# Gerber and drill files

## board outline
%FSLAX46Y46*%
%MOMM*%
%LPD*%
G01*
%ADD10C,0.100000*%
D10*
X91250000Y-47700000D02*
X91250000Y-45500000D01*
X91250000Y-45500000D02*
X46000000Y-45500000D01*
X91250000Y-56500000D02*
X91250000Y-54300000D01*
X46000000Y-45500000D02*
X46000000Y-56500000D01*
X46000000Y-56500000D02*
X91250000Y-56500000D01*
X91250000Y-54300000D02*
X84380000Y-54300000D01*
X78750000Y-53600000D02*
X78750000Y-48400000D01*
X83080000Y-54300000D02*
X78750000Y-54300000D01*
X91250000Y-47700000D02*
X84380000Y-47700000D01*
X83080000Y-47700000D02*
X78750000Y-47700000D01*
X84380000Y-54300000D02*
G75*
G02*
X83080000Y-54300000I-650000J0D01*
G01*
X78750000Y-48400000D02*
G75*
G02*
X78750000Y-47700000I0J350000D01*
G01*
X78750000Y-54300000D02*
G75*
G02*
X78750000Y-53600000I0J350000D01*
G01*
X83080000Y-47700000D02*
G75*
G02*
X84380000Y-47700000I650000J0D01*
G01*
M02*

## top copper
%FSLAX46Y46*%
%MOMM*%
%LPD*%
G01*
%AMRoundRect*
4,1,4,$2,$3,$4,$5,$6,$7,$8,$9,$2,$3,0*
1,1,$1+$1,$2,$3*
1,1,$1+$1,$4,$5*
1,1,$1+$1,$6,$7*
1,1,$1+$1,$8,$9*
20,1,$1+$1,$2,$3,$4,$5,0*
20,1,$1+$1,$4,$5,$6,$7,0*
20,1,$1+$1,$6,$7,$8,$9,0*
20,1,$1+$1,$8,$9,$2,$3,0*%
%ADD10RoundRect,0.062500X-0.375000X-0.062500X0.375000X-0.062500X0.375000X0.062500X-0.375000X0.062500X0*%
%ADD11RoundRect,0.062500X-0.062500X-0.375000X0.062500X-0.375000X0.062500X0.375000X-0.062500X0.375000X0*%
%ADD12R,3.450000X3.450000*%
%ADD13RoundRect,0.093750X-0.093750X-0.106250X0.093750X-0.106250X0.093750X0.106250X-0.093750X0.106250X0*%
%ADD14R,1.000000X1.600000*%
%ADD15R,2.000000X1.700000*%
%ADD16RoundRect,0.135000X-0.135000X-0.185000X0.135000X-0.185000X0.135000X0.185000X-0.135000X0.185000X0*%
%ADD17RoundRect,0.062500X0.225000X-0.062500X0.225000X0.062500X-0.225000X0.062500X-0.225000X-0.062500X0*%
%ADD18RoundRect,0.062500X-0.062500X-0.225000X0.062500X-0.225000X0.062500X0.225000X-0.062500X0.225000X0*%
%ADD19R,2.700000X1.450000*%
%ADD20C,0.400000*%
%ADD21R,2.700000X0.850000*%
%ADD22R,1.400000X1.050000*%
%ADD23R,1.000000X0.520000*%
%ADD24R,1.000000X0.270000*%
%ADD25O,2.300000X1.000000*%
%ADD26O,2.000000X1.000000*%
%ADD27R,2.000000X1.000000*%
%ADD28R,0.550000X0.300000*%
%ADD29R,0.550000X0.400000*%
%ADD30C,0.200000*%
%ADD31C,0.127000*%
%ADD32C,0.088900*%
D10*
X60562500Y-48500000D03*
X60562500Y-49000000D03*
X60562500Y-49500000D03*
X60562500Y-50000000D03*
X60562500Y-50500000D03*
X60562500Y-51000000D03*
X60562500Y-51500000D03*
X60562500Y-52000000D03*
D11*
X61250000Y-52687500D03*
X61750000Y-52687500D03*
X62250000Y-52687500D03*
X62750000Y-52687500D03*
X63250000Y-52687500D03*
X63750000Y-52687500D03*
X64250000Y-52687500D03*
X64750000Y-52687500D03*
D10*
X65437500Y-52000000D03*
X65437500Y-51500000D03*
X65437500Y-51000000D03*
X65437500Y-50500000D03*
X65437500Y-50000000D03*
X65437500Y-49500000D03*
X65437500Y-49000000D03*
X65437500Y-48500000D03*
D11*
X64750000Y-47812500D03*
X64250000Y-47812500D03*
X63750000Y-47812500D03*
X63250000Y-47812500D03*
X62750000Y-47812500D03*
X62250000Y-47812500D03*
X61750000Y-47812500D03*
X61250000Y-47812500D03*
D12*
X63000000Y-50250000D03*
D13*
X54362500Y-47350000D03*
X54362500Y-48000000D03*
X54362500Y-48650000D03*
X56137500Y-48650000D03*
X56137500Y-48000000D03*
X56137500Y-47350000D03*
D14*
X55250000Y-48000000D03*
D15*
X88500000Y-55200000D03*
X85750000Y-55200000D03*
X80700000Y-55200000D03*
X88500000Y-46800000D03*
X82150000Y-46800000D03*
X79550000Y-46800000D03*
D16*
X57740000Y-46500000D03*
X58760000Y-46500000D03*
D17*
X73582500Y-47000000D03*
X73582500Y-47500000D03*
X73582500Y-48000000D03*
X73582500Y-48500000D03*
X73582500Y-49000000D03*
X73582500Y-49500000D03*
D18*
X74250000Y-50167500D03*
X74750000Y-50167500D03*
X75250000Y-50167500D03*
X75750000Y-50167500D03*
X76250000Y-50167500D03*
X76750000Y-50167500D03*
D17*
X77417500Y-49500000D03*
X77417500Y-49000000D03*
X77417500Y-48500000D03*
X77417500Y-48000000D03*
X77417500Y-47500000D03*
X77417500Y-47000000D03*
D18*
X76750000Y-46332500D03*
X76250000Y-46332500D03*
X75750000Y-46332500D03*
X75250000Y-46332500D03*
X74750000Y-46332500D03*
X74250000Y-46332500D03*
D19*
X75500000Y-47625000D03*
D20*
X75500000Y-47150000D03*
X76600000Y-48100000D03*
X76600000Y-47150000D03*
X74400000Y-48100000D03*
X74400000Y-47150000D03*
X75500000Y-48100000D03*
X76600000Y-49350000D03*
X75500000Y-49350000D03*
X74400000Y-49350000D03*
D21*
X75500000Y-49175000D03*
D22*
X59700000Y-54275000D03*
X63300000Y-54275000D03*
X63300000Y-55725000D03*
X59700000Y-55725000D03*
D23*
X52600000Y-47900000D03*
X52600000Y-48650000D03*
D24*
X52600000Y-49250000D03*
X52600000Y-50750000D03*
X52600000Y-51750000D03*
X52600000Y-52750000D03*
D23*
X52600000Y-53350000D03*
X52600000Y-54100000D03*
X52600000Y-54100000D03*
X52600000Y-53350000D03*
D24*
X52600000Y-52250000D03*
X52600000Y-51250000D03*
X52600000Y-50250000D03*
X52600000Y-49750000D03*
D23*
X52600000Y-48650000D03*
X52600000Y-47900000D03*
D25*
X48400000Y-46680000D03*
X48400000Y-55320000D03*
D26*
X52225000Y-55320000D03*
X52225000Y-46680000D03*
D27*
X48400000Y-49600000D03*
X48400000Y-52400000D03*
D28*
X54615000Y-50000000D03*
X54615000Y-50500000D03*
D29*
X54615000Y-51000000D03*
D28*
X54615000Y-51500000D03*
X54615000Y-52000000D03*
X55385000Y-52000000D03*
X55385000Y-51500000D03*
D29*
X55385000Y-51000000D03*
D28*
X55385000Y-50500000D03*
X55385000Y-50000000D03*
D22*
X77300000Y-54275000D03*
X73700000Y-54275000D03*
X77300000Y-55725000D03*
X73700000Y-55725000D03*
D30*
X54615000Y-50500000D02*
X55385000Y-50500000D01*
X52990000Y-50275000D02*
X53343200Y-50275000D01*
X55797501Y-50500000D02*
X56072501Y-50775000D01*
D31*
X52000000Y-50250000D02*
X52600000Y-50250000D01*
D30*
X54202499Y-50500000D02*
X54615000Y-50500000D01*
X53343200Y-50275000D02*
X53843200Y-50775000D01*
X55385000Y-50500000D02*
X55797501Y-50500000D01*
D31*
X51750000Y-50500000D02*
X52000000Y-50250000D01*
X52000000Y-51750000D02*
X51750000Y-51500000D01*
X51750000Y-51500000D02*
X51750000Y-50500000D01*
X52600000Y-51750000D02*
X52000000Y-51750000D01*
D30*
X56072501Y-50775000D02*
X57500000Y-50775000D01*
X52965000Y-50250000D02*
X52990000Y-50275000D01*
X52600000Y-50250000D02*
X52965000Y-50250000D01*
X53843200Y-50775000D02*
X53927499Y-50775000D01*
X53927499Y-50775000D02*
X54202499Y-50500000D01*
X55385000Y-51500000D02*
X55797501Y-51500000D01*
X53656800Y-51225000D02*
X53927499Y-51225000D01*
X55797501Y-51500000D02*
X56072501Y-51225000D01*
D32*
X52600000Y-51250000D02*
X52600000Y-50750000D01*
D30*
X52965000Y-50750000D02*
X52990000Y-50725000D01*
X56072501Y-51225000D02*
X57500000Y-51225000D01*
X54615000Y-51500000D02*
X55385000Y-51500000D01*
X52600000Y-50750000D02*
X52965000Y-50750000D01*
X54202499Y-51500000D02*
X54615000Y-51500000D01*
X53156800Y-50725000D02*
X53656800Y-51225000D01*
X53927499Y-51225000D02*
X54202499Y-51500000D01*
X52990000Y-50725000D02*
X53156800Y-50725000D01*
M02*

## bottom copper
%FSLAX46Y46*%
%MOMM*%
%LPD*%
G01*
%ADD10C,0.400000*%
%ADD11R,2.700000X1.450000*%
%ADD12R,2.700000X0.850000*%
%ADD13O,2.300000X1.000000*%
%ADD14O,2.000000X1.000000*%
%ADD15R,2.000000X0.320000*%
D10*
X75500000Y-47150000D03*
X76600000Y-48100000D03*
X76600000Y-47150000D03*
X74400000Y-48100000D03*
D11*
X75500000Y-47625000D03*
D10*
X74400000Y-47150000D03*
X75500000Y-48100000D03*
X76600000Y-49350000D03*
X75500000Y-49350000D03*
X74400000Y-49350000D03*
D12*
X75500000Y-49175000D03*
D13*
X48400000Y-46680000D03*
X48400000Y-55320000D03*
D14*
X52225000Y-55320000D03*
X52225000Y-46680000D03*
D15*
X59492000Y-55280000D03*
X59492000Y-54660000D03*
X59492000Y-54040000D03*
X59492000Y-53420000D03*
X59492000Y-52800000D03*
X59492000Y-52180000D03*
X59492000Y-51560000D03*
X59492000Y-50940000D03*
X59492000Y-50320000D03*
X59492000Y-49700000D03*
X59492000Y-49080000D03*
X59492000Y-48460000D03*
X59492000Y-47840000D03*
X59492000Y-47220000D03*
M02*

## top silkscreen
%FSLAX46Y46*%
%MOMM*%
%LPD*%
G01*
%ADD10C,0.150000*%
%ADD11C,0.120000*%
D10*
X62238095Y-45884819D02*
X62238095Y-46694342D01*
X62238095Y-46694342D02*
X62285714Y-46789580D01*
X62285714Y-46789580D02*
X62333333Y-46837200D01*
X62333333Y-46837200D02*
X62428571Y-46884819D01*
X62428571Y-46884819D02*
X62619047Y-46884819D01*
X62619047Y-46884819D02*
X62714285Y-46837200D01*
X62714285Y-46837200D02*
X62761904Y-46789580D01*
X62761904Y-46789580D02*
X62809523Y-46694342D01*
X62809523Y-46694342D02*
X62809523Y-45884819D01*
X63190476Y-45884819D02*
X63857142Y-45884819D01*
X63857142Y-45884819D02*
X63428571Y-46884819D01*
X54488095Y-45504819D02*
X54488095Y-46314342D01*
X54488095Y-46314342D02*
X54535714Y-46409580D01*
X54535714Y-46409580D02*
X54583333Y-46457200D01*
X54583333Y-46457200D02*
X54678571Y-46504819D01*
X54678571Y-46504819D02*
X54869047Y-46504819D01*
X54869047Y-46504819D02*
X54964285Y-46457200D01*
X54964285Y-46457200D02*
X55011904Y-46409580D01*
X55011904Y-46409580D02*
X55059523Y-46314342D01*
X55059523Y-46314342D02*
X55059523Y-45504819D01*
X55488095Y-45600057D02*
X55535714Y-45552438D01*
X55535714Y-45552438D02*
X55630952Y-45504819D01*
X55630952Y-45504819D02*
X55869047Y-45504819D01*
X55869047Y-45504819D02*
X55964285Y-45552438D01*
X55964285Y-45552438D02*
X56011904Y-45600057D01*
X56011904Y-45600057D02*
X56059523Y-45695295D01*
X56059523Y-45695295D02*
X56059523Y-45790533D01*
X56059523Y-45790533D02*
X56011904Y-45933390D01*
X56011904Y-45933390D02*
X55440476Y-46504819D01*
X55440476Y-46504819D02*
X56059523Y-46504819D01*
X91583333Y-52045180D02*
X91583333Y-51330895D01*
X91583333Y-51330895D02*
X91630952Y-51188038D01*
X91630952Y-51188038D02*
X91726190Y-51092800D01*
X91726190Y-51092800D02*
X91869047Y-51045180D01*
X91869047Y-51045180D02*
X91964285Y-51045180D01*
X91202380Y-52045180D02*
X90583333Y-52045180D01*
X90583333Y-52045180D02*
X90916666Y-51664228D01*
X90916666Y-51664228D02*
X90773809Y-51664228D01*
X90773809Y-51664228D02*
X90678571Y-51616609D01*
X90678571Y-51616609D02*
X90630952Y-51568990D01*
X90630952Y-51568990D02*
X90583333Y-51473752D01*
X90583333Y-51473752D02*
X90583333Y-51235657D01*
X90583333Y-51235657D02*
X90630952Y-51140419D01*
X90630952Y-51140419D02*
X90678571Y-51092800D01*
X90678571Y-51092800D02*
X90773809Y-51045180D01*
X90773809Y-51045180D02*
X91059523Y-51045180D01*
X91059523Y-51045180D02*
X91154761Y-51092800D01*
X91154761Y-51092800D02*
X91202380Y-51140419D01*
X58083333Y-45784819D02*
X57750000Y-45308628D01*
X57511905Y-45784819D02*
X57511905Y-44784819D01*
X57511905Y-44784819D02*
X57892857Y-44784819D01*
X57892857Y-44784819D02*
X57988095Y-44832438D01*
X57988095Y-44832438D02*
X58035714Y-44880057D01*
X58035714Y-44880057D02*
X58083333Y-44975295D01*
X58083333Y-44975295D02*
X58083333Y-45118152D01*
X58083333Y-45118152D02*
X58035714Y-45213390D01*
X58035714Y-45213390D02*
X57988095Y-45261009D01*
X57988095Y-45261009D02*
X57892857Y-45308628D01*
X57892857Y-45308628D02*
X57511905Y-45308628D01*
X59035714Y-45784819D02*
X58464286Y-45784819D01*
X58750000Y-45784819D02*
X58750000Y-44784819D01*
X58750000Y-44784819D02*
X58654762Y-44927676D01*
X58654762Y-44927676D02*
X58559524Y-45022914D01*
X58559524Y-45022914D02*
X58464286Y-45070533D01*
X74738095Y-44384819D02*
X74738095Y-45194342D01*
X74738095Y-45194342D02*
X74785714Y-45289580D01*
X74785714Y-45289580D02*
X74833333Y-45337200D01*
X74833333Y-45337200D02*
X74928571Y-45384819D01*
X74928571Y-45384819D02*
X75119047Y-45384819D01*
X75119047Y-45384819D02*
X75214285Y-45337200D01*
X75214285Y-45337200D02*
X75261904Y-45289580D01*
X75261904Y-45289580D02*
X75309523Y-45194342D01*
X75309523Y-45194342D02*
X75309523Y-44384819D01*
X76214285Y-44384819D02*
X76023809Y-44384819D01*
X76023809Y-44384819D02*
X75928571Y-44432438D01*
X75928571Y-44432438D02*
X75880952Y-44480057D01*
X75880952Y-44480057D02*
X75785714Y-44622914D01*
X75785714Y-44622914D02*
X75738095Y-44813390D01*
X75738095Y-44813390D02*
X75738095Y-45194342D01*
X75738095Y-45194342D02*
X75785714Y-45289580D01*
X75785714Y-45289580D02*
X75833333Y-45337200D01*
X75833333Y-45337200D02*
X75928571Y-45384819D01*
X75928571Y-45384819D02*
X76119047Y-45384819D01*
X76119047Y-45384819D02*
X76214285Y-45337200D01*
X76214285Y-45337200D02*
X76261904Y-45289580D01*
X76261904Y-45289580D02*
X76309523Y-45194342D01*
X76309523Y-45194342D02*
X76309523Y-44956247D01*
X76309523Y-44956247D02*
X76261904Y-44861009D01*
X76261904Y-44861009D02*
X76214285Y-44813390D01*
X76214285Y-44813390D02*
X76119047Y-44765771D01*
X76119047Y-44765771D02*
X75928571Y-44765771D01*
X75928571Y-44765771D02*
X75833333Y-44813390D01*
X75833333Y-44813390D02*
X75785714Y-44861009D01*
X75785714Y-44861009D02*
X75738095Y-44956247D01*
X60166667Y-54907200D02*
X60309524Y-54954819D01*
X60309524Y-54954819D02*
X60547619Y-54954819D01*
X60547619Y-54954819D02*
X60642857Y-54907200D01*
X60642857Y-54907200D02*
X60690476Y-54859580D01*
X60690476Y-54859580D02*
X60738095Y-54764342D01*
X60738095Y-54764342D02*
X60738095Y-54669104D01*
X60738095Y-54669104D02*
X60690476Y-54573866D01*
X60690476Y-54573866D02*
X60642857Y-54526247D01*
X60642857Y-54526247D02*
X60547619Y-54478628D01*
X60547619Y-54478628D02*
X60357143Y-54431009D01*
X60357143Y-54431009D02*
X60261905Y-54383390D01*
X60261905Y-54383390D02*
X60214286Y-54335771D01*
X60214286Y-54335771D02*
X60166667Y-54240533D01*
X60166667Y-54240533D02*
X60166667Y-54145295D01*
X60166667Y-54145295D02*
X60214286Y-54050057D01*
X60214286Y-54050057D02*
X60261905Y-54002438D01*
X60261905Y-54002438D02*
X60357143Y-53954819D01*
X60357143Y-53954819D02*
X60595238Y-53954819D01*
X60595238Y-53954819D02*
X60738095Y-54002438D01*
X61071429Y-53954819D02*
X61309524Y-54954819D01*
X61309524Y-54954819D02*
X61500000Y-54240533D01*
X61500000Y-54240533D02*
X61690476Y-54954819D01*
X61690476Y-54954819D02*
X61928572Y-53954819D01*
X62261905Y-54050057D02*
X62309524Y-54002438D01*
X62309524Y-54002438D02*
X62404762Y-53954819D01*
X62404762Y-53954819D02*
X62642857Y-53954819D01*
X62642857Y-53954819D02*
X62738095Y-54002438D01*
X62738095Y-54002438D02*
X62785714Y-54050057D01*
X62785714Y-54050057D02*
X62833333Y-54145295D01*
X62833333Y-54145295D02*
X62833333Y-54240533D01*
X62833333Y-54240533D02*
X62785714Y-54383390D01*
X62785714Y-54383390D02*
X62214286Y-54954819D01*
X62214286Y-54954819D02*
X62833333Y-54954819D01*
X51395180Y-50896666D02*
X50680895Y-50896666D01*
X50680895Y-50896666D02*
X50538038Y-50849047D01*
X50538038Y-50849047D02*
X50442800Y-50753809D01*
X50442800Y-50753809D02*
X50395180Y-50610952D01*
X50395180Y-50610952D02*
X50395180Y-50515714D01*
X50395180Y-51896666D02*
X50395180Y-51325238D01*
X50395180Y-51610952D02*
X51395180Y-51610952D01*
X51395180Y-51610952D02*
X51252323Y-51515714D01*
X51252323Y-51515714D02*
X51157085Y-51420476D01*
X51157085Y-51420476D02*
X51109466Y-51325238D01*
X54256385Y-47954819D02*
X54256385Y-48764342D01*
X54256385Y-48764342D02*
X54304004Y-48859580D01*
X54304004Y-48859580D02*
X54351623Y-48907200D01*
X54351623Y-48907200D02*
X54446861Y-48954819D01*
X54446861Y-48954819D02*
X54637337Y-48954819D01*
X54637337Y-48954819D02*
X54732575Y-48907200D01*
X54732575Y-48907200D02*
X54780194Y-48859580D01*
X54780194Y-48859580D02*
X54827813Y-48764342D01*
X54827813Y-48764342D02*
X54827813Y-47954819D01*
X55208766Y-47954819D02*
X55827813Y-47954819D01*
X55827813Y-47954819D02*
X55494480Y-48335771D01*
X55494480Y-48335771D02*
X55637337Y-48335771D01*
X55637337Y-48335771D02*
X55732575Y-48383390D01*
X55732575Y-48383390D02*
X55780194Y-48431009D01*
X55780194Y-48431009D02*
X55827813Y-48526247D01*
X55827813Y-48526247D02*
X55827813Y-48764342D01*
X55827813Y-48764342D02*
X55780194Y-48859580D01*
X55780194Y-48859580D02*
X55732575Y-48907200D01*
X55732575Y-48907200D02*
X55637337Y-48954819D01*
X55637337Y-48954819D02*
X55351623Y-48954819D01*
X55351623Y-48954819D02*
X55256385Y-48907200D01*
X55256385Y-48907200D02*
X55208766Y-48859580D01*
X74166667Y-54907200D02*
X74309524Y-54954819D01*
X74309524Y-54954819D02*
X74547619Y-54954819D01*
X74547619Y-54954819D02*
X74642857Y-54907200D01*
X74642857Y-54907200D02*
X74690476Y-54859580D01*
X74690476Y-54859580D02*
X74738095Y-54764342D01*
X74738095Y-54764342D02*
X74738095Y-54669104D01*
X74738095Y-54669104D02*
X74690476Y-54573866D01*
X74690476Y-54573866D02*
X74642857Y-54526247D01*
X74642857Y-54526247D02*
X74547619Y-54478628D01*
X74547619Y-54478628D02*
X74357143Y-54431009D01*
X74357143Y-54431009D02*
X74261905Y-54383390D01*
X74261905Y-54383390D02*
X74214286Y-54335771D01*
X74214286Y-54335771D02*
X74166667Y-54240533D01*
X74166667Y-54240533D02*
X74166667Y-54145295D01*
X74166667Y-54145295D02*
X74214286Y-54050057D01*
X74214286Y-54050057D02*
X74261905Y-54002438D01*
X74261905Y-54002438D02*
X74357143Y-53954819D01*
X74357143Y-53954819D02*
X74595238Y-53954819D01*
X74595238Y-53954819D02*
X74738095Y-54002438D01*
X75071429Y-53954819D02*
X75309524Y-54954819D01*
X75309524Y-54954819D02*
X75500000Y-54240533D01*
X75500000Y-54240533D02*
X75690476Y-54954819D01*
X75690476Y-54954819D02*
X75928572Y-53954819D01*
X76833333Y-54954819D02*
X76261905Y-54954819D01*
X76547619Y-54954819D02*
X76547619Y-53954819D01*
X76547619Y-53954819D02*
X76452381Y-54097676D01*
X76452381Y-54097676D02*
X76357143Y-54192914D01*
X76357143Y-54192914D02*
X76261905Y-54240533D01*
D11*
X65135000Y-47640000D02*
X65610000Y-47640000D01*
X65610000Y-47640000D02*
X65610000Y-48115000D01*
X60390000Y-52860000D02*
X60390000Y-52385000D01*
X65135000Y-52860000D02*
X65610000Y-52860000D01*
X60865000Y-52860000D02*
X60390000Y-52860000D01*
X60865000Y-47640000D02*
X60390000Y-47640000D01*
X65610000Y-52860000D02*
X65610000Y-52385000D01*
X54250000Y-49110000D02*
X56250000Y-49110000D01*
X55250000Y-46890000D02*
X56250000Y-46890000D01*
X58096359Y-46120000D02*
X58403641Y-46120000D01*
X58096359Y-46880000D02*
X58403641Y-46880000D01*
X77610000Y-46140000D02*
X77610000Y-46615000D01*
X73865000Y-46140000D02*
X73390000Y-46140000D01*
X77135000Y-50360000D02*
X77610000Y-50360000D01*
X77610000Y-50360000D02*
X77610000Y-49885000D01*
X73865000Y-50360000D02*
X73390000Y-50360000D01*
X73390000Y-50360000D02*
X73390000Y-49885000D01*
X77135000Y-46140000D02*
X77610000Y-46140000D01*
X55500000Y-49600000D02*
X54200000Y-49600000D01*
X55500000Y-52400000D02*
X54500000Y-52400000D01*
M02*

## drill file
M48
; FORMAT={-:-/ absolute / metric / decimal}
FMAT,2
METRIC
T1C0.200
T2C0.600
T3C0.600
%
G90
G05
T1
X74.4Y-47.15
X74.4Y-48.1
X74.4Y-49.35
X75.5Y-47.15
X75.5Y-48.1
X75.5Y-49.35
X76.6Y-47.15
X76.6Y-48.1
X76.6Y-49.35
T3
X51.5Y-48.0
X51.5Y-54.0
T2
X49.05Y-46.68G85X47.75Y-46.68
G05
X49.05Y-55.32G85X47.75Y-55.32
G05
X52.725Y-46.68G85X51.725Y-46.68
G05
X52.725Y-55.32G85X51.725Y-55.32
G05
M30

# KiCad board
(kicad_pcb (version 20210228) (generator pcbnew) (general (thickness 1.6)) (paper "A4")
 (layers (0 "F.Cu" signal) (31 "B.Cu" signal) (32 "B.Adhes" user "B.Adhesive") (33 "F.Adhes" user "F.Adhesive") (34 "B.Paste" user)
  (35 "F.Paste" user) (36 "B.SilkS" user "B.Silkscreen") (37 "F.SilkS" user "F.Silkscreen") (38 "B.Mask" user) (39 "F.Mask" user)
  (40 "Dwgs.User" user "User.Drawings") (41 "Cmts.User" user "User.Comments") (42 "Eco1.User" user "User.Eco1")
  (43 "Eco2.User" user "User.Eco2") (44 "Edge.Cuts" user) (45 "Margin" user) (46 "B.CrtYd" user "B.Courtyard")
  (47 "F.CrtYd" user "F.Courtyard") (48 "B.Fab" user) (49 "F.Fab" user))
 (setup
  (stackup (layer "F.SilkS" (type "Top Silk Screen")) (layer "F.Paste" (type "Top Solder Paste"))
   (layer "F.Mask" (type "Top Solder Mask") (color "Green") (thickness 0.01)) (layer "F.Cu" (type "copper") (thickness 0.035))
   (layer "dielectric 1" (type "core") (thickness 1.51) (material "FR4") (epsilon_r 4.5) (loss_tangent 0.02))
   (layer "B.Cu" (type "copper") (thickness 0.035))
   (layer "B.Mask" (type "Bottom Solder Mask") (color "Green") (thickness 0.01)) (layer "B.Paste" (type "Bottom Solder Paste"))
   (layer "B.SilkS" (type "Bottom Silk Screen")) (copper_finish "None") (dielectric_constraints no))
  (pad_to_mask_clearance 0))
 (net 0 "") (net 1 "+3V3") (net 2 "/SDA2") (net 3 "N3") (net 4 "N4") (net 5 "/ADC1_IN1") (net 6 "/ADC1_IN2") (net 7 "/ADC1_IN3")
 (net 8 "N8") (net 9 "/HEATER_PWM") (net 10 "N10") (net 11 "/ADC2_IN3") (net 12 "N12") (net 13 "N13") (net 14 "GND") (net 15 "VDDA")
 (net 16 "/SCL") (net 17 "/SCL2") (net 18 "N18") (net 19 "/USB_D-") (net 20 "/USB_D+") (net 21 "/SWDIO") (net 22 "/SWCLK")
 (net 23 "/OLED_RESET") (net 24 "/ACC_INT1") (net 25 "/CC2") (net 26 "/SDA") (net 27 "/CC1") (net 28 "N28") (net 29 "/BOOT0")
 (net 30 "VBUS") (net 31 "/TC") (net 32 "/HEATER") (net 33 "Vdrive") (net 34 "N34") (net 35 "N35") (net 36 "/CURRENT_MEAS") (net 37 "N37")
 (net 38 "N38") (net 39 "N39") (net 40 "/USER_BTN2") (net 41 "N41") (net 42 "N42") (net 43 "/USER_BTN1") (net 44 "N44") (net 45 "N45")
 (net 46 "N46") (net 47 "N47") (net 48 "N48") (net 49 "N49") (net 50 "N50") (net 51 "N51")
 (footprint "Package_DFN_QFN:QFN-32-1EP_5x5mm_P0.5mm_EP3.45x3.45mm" (layer "F.Cu") (at 63 50.25)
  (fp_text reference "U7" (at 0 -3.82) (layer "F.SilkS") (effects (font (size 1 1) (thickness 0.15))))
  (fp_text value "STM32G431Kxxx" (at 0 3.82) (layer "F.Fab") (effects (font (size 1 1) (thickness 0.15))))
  (fp_line (start 2.135 -2.61) (end 2.61 -2.61) (layer "F.SilkS") (width 0.12))
  (fp_line (start 2.61 -2.61) (end 2.61 -2.135) (layer "F.SilkS") (width 0.12))
  (fp_line (start -2.61 2.61) (end -2.61 2.135) (layer "F.SilkS") (width 0.12))
  (fp_line (start 2.135 2.61) (end 2.61 2.61) (layer "F.SilkS") (width 0.12))
  (fp_line (start -2.135 2.61) (end -2.61 2.61) (layer "F.SilkS") (width 0.12))
  (fp_line (start -2.135 -2.61) (end -2.61 -2.61) (layer "F.SilkS") (width 0.12))
  (fp_line (start 2.61 2.61) (end 2.61 2.135) (layer "F.SilkS") (width 0.12))
  (pad "" smd roundrect (at -1.15 0) (locked) (size 0.93 0.93) (layers "F.Paste") (roundrect_rratio 0.25))
  (pad "" smd roundrect (at -1.15 -1.15) (locked) (size 0.93 0.93) (layers "F.Paste") (roundrect_rratio 0.25))
  (pad "" smd roundrect (at 0 1.15) (locked) (size 0.93 0.93) (layers "F.Paste") (roundrect_rratio 0.25))
  (pad "" smd roundrect (at 1.15 0) (locked) (size 0.93 0.93) (layers "F.Paste") (roundrect_rratio 0.25))
  (pad "" smd roundrect (at 0 0) (locked) (size 0.93 0.93) (layers "F.Paste") (roundrect_rratio 0.25))
  (pad "" smd roundrect (at -1.15 1.15) (locked) (size 0.93 0.93) (layers "F.Paste") (roundrect_rratio 0.25))
  (pad "" smd roundrect (at 0 -1.15) (locked) (size 0.93 0.93) (layers "F.Paste") (roundrect_rratio 0.25))
  (pad "" smd roundrect (at 1.15 1.15) (locked) (size 0.93 0.93) (layers "F.Paste") (roundrect_rratio 0.25))
  (pad "" smd roundrect (at 1.15 -1.15) (locked) (size 0.93 0.93) (layers "F.Paste") (roundrect_rratio 0.25))
  (pad "1" smd roundrect (at -2.4375 -1.75) (locked) (size 0.875 0.25) (layers "F.Cu" "F.Paste" "F.Mask") (roundrect_rratio 0.25)
   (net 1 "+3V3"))
  (pad "2" smd roundrect (at -2.4375 -1.25) (locked) (size 0.875 0.25) (layers "F.Cu" "F.Paste" "F.Mask") (roundrect_rratio 0.25)
   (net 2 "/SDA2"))
  (pad "3" smd roundrect (at -2.4375 -0.75) (locked) (size 0.875 0.25) (layers "F.Cu" "F.Paste" "F.Mask") (roundrect_rratio 0.25)
   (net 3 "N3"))
  (pad "4" smd roundrect (at -2.4375 -0.25) (locked) (size 0.875 0.25) (layers "F.Cu" "F.Paste" "F.Mask") (roundrect_rratio 0.25)
   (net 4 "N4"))
  (pad "5" smd roundrect (at -2.4375 0.25) (locked) (size 0.875 0.25) (layers "F.Cu" "F.Paste" "F.Mask") (roundrect_rratio 0.25)
   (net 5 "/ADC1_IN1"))
  (pad "6" smd roundrect (at -2.4375 0.75) (locked) (size 0.875 0.25) (layers "F.Cu" "F.Paste" "F.Mask") (roundrect_rratio 0.25)
   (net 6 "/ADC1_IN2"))
  (pad "7" smd roundrect (at -2.4375 1.25) (locked) (size 0.875 0.25) (layers "F.Cu" "F.Paste" "F.Mask") (roundrect_rratio 0.25)
   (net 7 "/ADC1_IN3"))
  (pad "8" smd roundrect (at -2.4375 1.75) (locked) (size 0.875 0.25) (layers "F.Cu" "F.Paste" "F.Mask") (roundrect_rratio 0.25)
   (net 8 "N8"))
  (pad "9" smd roundrect (at -1.75 2.4375) (locked) (size 0.25 0.875) (layers "F.Cu" "F.Paste" "F.Mask") (roundrect_rratio 0.25)
   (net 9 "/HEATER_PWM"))
  (pad "10" smd roundrect (at -1.25 2.4375) (locked) (size 0.25 0.875) (layers "F.Cu" "F.Paste" "F.Mask") (roundrect_rratio 0.25)
   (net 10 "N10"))
  (pad "11" smd roundrect (at -0.75 2.4375) (locked) (size 0.25 0.875) (layers "F.Cu" "F.Paste" "F.Mask") (roundrect_rratio 0.25)
   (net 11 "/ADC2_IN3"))
  (pad "12" smd roundrect (at -0.25 2.4375) (locked) (size 0.25 0.875) (layers "F.Cu" "F.Paste" "F.Mask") (roundrect_rratio 0.25)
   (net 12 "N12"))
  (pad "13" smd roundrect (at 0.25 2.4375) (locked) (size 0.25 0.875) (layers "F.Cu" "F.Paste" "F.Mask") (roundrect_rratio 0.25)
   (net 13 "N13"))
  (pad "14" smd roundrect (at 0.75 2.4375) (locked) (size 0.25 0.875) (layers "F.Cu" "F.Paste" "F.Mask") (roundrect_rratio 0.25)
   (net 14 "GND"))
  (pad "15" smd roundrect (at 1.25 2.4375) (locked) (size 0.25 0.875) (layers "F.Cu" "F.Paste" "F.Mask") (roundrect_rratio 0.25)
   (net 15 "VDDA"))
  (pad "16" smd roundrect (at 1.75 2.4375) (locked) (size 0.25 0.875) (layers "F.Cu" "F.Paste" "F.Mask") (roundrect_rratio 0.25)
   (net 14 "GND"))
  (pad "17" smd roundrect (at 2.4375 1.75) (locked) (size 0.875 0.25) (layers "F.Cu" "F.Paste" "F.Mask") (roundrect_rratio 0.25)
   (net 1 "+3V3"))
  (pad "18" smd roundrect (at 2.4375 1.25) (locked) (size 0.875 0.25) (layers "F.Cu" "F.Paste" "F.Mask") (roundrect_rratio 0.25)
   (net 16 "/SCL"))
  (pad "19" smd roundrect (at 2.4375 0.75) (locked) (size 0.875 0.25) (layers "F.Cu" "F.Paste" "F.Mask") (roundrect_rratio 0.25)
   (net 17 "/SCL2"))
  (pad "20" smd roundrect (at 2.4375 0.25) (locked) (size 0.875 0.25) (layers "F.Cu" "F.Paste" "F.Mask") (roundrect_rratio 0.25)
   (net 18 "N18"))
  (pad "21" smd roundrect (at 2.4375 -0.25) (locked) (size 0.875 0.25) (layers "F.Cu" "F.Paste" "F.Mask") (roundrect_rratio 0.25)
   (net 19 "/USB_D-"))
  (pad "22" smd roundrect (at 2.4375 -0.75) (locked) (size 0.875 0.25) (layers "F.Cu" "F.Paste" "F.Mask") (roundrect_rratio 0.25)
   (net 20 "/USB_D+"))
  (pad "23" smd roundrect (at 2.4375 -1.25) (locked) (size 0.875 0.25) (layers "F.Cu" "F.Paste" "F.Mask") (roundrect_rratio 0.25)
   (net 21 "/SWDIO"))
  (pad "24" smd roundrect (at 2.4375 -1.75) (locked) (size 0.875 0.25) (layers "F.Cu" "F.Paste" "F.Mask") (roundrect_rratio 0.25)
   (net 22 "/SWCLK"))
  (pad "25" smd roundrect (at 1.75 -2.4375) (locked) (size 0.25 0.875) (layers "F.Cu" "F.Paste" "F.Mask") (roundrect_rratio 0.25)
   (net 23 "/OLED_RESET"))
  (pad "26" smd roundrect (at 1.25 -2.4375) (locked) (size 0.25 0.875) (layers "F.Cu" "F.Paste" "F.Mask") (roundrect_rratio 0.25)
   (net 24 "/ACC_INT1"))
  (pad "27" smd roundrect (at 0.75 -2.4375) (locked) (size 0.25 0.875) (layers "F.Cu" "F.Paste" "F.Mask") (roundrect_rratio 0.25)
   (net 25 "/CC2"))
  (pad "28" smd roundrect (at 0.25 -2.4375) (locked) (size 0.25 0.875) (layers "F.Cu" "F.Paste" "F.Mask") (roundrect_rratio 0.25)
   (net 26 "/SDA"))
  (pad "29" smd roundrect (at -0.25 -2.4375) (locked) (size 0.25 0.875) (layers "F.Cu" "F.Paste" "F.Mask") (roundrect_rratio 0.25)
   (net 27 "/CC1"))
  (pad "30" smd roundrect (at -0.75 -2.4375) (locked) (size 0.25 0.875) (layers "F.Cu" "F.Paste" "F.Mask") (roundrect_rratio 0.25)
   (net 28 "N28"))
  (pad "31" smd roundrect (at -1.25 -2.4375) (locked) (size 0.25 0.875) (layers "F.Cu" "F.Paste" "F.Mask") (roundrect_rratio 0.25)
   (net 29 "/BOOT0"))
  (pad "32" smd roundrect (at -1.75 -2.4375) (locked) (size 0.25 0.875) (layers "F.Cu" "F.Paste" "F.Mask") (roundrect_rratio 0.25)
   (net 14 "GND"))
  (pad "33" smd rect (at 0 0) (locked) (size 3.45 3.45) (layers "F.Cu" "F.Mask") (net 14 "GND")))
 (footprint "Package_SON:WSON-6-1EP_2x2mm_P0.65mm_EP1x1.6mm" (layer "F.Cu") (at 55.25 48)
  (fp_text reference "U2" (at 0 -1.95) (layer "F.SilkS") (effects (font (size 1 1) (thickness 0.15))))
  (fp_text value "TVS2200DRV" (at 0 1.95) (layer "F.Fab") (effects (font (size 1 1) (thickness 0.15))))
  (fp_line (start -1 1.11) (end 1 1.11) (layer "F.SilkS") (width 0.12))
  (fp_line (start 0 -1.11) (end 1 -1.11) (layer "F.SilkS") (width 0.12))
  (pad "" smd roundrect (at 0 0.4) (locked) (size 0.81 0.64) (layers "F.Paste") (roundrect_rratio 0.25))
  (pad "" smd roundrect (at 0 -0.4) (locked) (size 0.81 0.64) (layers "F.Paste") (roundrect_rratio 0.25))
  (pad "1" smd roundrect (at -0.8875 -0.65) (locked) (size 0.375 0.4) (layers "F.Cu" "F.Paste" "F.Mask") (roundrect_rratio 0.25)
   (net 14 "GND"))
  (pad "2" smd roundrect (at -0.8875 0) (locked) (size 0.375 0.4) (layers "F.Cu" "F.Paste" "F.Mask") (roundrect_rratio 0.25) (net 14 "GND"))
  (pad "3" smd roundrect (at -0.8875 0.65) (locked) (size 0.375 0.4) (layers "F.Cu" "F.Paste" "F.Mask") (roundrect_rratio 0.25)
   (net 14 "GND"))
  (pad "4" smd roundrect (at 0.8875 0.65) (locked) (size 0.375 0.4) (layers "F.Cu" "F.Paste" "F.Mask") (roundrect_rratio 0.25)
   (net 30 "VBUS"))
  (pad "5" smd roundrect (at 0.8875 0) (locked) (size 0.375 0.4) (layers "F.Cu" "F.Paste" "F.Mask") (roundrect_rratio 0.25) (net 30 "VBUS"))
  (pad "6" smd roundrect (at 0.8875 -0.65) (locked) (size 0.375 0.4) (layers "F.Cu" "F.Paste" "F.Mask") (roundrect_rratio 0.25)
   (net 30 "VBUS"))
  (pad "7" smd rect (at 0 0) (locked) (size 1 1.6) (layers "F.Cu" "F.Mask") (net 14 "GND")))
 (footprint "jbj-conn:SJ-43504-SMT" (layer "F.Cu") (at 91.25 51 180)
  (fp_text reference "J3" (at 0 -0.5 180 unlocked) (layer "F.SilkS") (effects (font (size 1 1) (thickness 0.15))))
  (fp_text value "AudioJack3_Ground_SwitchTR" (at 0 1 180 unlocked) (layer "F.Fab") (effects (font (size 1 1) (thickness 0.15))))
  (fp_line (start 0 -3.3) (end 6.87 -3.3) (layer "Edge.Cuts") (width 0.1))
  (fp_line (start 12.5 -2.6) (end 12.5 2.6) (layer "Edge.Cuts") (width 0.1))
  (fp_line (start 8.17 -3.3) (end 12.5 -3.3) (layer "Edge.Cuts") (width 0.1))
  (fp_line (start 0 3.3) (end 6.87 3.3) (layer "Edge.Cuts") (width 0.1))
  (fp_line (start 8.17 3.3) (end 12.5 3.3) (layer "Edge.Cuts") (width 0.1))
  (fp_arc (start 7.52 -3.3) (end 6.87 -3.3) (angle 180) (layer "Edge.Cuts") (width 0.1))
  (fp_arc (start 12.5 2.95) (end 12.5 3.3) (angle -180) (layer "Edge.Cuts") (width 0.1))
  (fp_arc (start 12.5 -2.95) (end 12.5 -3.3) (angle 180) (layer "Edge.Cuts") (width 0.1))
  (fp_arc (start 7.52 3.3) (end 6.87 3.3) (angle -180) (layer "Edge.Cuts") (width 0.1))
  (pad "G" smd rect (at 2.75 -4.2 180) (locked) (size 2 1.7) (layers "F.Cu" "F.Paste" "F.Mask") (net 14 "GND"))
  (pad "R" smd rect (at 5.5 -4.2 180) (locked) (size 2 1.7) (layers "F.Cu" "F.Paste" "F.Mask") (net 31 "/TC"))
  (pad "RN" smd rect (at 10.55 -4.2 180) (locked) (size 2 1.7) (layers "F.Cu" "F.Paste" "F.Mask") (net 31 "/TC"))
  (pad "S" smd rect (at 2.75 4.2 180) (locked) (size 2 1.7) (layers "F.Cu" "F.Paste" "F.Mask") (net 14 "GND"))
  (pad "T" smd rect (at 9.1 4.2 180) (locked) (size 2 1.7) (layers "F.Cu" "F.Paste" "F.Mask") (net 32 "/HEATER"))
  (pad "TN" smd rect (at 11.7 4.2 180) (locked) (size 2 1.7) (layers "F.Cu" "F.Paste" "F.Mask") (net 32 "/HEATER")))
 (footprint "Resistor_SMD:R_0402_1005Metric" (layer "F.Cu") (at 58.25 46.5)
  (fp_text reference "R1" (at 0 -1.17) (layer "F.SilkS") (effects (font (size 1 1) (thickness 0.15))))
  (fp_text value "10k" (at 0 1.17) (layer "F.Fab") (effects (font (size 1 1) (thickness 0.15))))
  (fp_line (start -0.153641 -0.38) (end 0.153641 -0.38) (layer "F.SilkS") (width 0.12))
  (fp_line (start -0.153641 0.38) (end 0.153641 0.38) (layer "F.SilkS") (width 0.12))
  (pad "1" smd roundrect (at -0.51 0) (locked) (size 0.54 0.64) (layers "F.Cu" "F.Paste" "F.Mask") (roundrect_rratio 0.25)
   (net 6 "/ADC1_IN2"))
  (pad "2" smd roundrect (at 0.51 0) (locked) (size 0.54 0.64) (layers "F.Cu" "F.Paste" "F.Mask") (roundrect_rratio 0.25) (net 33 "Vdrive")))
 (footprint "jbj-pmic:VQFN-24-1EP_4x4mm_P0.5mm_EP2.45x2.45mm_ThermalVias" (layer "F.Cu") (at 75.5 48.25)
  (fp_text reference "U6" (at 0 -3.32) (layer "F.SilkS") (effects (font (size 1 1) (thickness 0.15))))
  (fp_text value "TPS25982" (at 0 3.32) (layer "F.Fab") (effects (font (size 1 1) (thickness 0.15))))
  (fp_line (start 2.11 -2.11) (end 2.11 -1.635) (layer "F.SilkS") (width 0.12))
  (fp_line (start -1.635 -2.11) (end -2.11 -2.11) (layer "F.SilkS") (width 0.12))
  (fp_line (start 1.635 2.11) (end 2.11 2.11) (layer "F.SilkS") (width 0.12))
  (fp_line (start 2.11 2.11) (end 2.11 1.635) (layer "F.SilkS") (width 0.12))
  (fp_line (start -1.635 2.11) (end -2.11 2.11) (layer "F.SilkS") (width 0.12))
  (fp_line (start -2.11 2.11) (end -2.11 1.635) (layer "F.SilkS") (width 0.12))
  (fp_line (start 1.635 -2.11) (end 2.11 -2.11) (layer "F.SilkS") (width 0.12))
  (pad "" smd roundrect (at -0.694 -0.625) (locked) (size 1.188 1.3) (layers "F.Paste") (roundrect_rratio 0.132))
  (pad "" smd roundrect (at 0.694 0.925) (locked) (size 1.188 0.76) (layers "F.Paste") (roundrect_rratio 0.132))
  (pad "" smd roundrect (at 0.694 -0.625) (locked) (size 1.188 1.3) (layers "F.Paste") (roundrect_rratio 0.132))
  (pad "" smd roundrect (at -0.694 0.925) (locked) (size 1.188 0.76) (layers "F.Paste") (roundrect_rratio 0.132))
  (pad "1" smd roundrect (at -1.9175 -1.25 90) (locked) (size 0.25 0.575) (layers "F.Cu" "F.Paste" "F.Mask") (roundrect_rratio 0.25)
   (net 33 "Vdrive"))
  (pad "2" smd roundrect (at -1.9175 -0.75 90) (locked) (size 0.25 0.575) (layers "F.Cu" "F.Paste" "F.Mask") (roundrect_rratio 0.25)
   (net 33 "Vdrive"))
  (pad "3" smd roundrect (at -1.9175 -0.25 90) (locked) (size 0.25 0.575) (layers "F.Cu" "F.Paste" "F.Mask") (roundrect_rratio 0.25)
   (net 33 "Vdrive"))
  (pad "4" smd roundrect (at -1.9175 0.25 90) (locked) (size 0.25 0.575) (layers "F.Cu" "F.Paste" "F.Mask") (roundrect_rratio 0.25)
   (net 14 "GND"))
  (pad "5" smd roundrect (at -1.9175 0.75 90) (locked) (size 0.25 0.575) (layers "F.Cu" "F.Paste" "F.Mask") (roundrect_rratio 0.25)
   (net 14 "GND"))
  (pad "6" smd roundrect (at -1.9175 1.25 90) (locked) (size 0.25 0.575) (layers "F.Cu" "F.Paste" "F.Mask") (roundrect_rratio 0.25)
   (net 9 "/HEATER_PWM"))
  (pad "7" smd roundrect (at -1.25 1.9175) (locked) (size 0.25 0.575) (layers "F.Cu" "F.Paste" "F.Mask") (roundrect_rratio 0.25)
   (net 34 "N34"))
  (pad "8" smd roundrect (at -0.75 1.9175) (locked) (size 0.25 0.575) (layers "F.Cu" "F.Paste" "F.Mask") (roundrect_rratio 0.25)
   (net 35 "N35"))
  (pad "9" smd roundrect (at -0.25 1.9175) (locked) (size 0.25 0.575) (layers "F.Cu" "F.Paste" "F.Mask") (roundrect_rratio 0.25)
   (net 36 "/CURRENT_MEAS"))
  (pad "10" smd roundrect (at 0.25 1.9175) (locked) (size 0.25 0.575) (layers "F.Cu" "F.Paste" "F.Mask") (roundrect_rratio 0.25)
   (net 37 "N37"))
  (pad "11" smd roundrect (at 0.75 1.9175) (locked) (size 0.25 0.575) (layers "F.Cu" "F.Paste" "F.Mask") (roundrect_rratio 0.25)
   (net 14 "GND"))
  (pad "12" smd roundrect (at 1.25 1.9175) (locked) (size 0.25 0.575) (layers "F.Cu" "F.Paste" "F.Mask") (roundrect_rratio 0.25)
   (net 14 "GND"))
  (pad "13" smd roundrect (at 1.9175 1.25 90) (locked) (size 0.25 0.575) (layers "F.Cu" "F.Paste" "F.Mask") (roundrect_rratio 0.25)
   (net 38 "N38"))
  (pad "14" smd roundrect (at 1.9175 0.75 90) (locked) (size 0.25 0.575) (layers "F.Cu" "F.Paste" "F.Mask") (roundrect_rratio 0.25)
   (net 14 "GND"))
  (pad "15" smd roundrect (at 1.9175 0.25 90) (locked) (size 0.25 0.575) (layers "F.Cu" "F.Paste" "F.Mask") (roundrect_rratio 0.25)
   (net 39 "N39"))
  (pad "16" smd roundrect (at 1.9175 -0.25 90) (locked) (size 0.25 0.575) (layers "F.Cu" "F.Paste" "F.Mask") (roundrect_rratio 0.25)
   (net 33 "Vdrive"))
  (pad "17" smd roundrect (at 1.9175 -0.75 90) (locked) (size 0.25 0.575) (layers "F.Cu" "F.Paste" "F.Mask") (roundrect_rratio 0.25)
   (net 32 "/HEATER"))
  (pad "18" smd roundrect (at 1.9175 -1.25 90) (locked) (size 0.25 0.575) (layers "F.Cu" "F.Paste" "F.Mask") (roundrect_rratio 0.25)
   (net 32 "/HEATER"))
  (pad "19" smd roundrect (at 1.25 -1.9175) (locked) (size 0.25 0.575) (layers "F.Cu" "F.Paste" "F.Mask") (roundrect_rratio 0.25)
   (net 32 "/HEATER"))
  (pad "20" smd roundrect (at 0.75 -1.9175) (locked) (size 0.25 0.575) (layers "F.Cu" "F.Paste" "F.Mask") (roundrect_rratio 0.25)
   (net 32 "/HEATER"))
  (pad "21" smd roundrect (at 0.25 -1.9175) (locked) (size 0.25 0.575) (layers "F.Cu" "F.Paste" "F.Mask") (roundrect_rratio 0.25)
   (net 32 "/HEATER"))
  (pad "22" smd roundrect (at -0.25 -1.9175) (locked) (size 0.25 0.575) (layers "F.Cu" "F.Paste" "F.Mask") (roundrect_rratio 0.25)
   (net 32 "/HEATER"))
  (pad "23" smd roundrect (at -0.75 -1.9175) (locked) (size 0.25 0.575) (layers "F.Cu" "F.Paste" "F.Mask") (roundrect_rratio 0.25)
   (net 32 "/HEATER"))
  (pad "24" smd roundrect (at -1.25 -1.9175) (locked) (size 0.25 0.575) (layers "F.Cu" "F.Paste" "F.Mask") (roundrect_rratio 0.25)
   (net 32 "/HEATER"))
  (pad "25" smd rect (at 0 -0.625) (locked) (size 2.7 1.45) (layers "F.Cu" "F.Mask") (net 33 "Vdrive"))
  (pad "25" thru_hole circle (at 0 -1.1) (locked) (size 0.4 0.4) (drill 0.2) (layers *.Cu) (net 33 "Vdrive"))
  (pad "25" thru_hole circle (at 1.1 -0.15) (locked) (size 0.4 0.4) (drill 0.2) (layers *.Cu) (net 33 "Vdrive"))
  (pad "25" thru_hole circle (at 1.1 -1.1) (locked) (size 0.4 0.4) (drill 0.2) (layers *.Cu) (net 33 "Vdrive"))
  (pad "25" thru_hole circle (at -1.1 -0.15) (locked) (size 0.4 0.4) (drill 0.2) (layers *.Cu) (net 33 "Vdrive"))
  (pad "25" smd rect (at 0 -0.625) (locked) (size 2.7 1.45) (layers "B.Cu" "B.Mask") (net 33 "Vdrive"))
  (pad "25" thru_hole circle (at -1.1 -1.1) (locked) (size 0.4 0.4) (drill 0.2) (layers *.Cu) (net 33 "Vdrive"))
  (pad "25" thru_hole circle (at 0 -0.15) (locked) (size 0.4 0.4) (drill 0.2) (layers *.Cu) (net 33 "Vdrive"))
  (pad "26" thru_hole circle (at 1.1 1.1) (locked) (size 0.4 0.4) (drill 0.2) (layers *.Cu) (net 14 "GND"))
  (pad "26" thru_hole circle (at 0 1.1) (locked) (size 0.4 0.4) (drill 0.2) (layers *.Cu) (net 14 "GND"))
  (pad "26" thru_hole circle (at -1.1 1.1) (locked) (size 0.4 0.4) (drill 0.2) (layers *.Cu) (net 14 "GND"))
  (pad "26" smd rect (at 0 0.925) (locked) (size 2.7 0.85) (layers "F.Cu" "F.Mask") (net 14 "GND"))
  (pad "26" smd rect (at 0 0.925) (locked) (size 2.7 0.85) (layers "B.Cu" "B.Mask") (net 14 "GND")))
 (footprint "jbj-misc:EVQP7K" (layer "F.Cu") (at 61.5 55)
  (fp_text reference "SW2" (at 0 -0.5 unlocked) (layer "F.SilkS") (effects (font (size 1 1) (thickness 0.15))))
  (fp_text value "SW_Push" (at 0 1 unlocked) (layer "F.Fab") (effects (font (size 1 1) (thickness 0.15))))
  (pad "1" smd rect (at -1.8 -0.725) (locked) (size 1.4 1.05) (layers "F.Cu" "F.Paste" "F.Mask") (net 1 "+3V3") (clearance 0.01))
  (pad "1" smd rect (at 1.8 -0.725) (locked) (size 1.4 1.05) (layers "F.Cu" "F.Paste" "F.Mask") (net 1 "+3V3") (clearance 0.01))
  (pad "2" smd rect (at 1.8 0.725) (locked) (size 1.4 1.05) (layers "F.Cu" "F.Paste" "F.Mask") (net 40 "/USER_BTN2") (clearance 0.01))
  (pad "2" smd rect (at -1.8 0.725) (locked) (size 1.4 1.05) (layers "F.Cu" "F.Paste" "F.Mask") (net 40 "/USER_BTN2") (clearance 0.01)))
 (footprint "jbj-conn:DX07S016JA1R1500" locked (layer "F.Cu") (at 51.5 51 -90)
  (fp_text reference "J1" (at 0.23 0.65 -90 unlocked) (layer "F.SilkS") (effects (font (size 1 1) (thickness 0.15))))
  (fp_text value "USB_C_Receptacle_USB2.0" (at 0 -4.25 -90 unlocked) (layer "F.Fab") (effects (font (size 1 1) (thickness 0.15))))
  (pad "" np_thru_hole circle (at 3 0 270) (locked) (size 0.65 0.65) (drill 0.6) (layers *.Mask) (clearance 0.01))
  (pad "" np_thru_hole circle (at -3 0 270) (locked) (size 0.65 0.65) (drill 0.6) (layers *.Mask) (clearance 0.01))
  (pad "A1" smd rect (at -3.1 -1.1 270) (locked) (size 0.52 1) (layers "F.Cu" "F.Paste" "F.Mask") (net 14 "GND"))
  (pad "A4" smd rect (at -2.35 -1.1 270) (locked) (size 0.52 1) (layers "F.Cu" "F.Paste" "F.Mask") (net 30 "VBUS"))
  (pad "A5" smd rect (at -1.75 -1.1 270) (locked) (size 0.27 1) (layers "F.Cu" "F.Paste" "F.Mask") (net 27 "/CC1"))
  (pad "A6" smd rect (at -0.25 -1.1 270) (locked) (size 0.27 1) (layers "F.Cu" "F.Paste" "F.Mask") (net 20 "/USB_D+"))
  (pad "A7" smd rect (at 0.75 -1.1 270) (locked) (size 0.27 1) (layers "F.Cu" "F.Paste" "F.Mask") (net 19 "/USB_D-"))
  (pad "A8" smd rect (at 1.75 -1.1 270) (locked) (size 0.27 1) (layers "F.Cu" "F.Paste" "F.Mask") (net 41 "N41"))
  (pad "A9" smd rect (at 2.35 -1.1 270) (locked) (size 0.52 1) (layers "F.Cu" "F.Paste" "F.Mask") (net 30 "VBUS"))
  (pad "A12" smd rect (at 3.1 -1.1 270) (locked) (size 0.52 1) (layers "F.Cu" "F.Paste" "F.Mask") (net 14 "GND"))
  (pad "B1" smd rect (at 3.1 -1.1 270) (locked) (size 0.52 1) (layers "F.Cu" "F.Paste" "F.Mask") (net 14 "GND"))
  (pad "B4" smd rect (at 2.35 -1.1 270) (locked) (size 0.52 1) (layers "F.Cu" "F.Paste" "F.Mask") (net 30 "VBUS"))
  (pad "B5" smd rect (at 1.25 -1.1 270) (locked) (size 0.27 1) (layers "F.Cu" "F.Paste" "F.Mask") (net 25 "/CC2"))
  (pad "B6" smd rect (at 0.25 -1.1 270) (locked) (size 0.27 1) (layers "F.Cu" "F.Paste" "F.Mask") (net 20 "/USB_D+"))
  (pad "B7" smd rect (at -0.75 -1.1 270) (locked) (size 0.27 1) (layers "F.Cu" "F.Paste" "F.Mask") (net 19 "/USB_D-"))
  (pad "B8" smd rect (at -1.25 -1.1 270) (locked) (size 0.27 1) (layers "F.Cu" "F.Paste" "F.Mask") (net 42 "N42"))
  (pad "B9" smd rect (at -2.35 -1.1 270) (locked) (size 0.52 1) (layers "F.Cu" "F.Paste" "F.Mask") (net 30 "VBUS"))
  (pad "B12" smd rect (at -3.1 -1.1 270) (locked) (size 0.52 1) (layers "F.Cu" "F.Paste" "F.Mask") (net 14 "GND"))
  (pad "S1" thru_hole oval (at -4.32 3.1 270) (locked) (size 1 2.3) (drill oval 0.6 1.9) (layers *.Cu *.Mask) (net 14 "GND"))
  (pad "S1" thru_hole oval (at 4.32 3.1 270) (locked) (size 1 2.3) (drill oval 0.6 1.9) (layers *.Cu *.Mask) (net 14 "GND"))
  (pad "S1" thru_hole oval (at 4.32 -0.725 270) (locked) (size 1 2) (drill oval 0.6 1.6) (layers *.Cu *.Mask) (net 14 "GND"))
  (pad "S1" thru_hole oval (at -4.32 -0.725 270) (locked) (size 1 2) (drill oval 0.6 1.6) (layers *.Cu *.Mask) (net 14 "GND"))
  (pad "S2" smd rect (at -1.4 3.1 270) (locked) (size 1 2) (layers "F.Cu" "F.Paste" "F.Mask"))
  (pad "S2" smd rect (at 1.4 3.1 270) (locked) (size 1 2) (layers "F.Cu" "F.Paste" "F.Mask")))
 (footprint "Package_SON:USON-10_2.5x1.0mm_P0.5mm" (layer "F.Cu") (at 55 51)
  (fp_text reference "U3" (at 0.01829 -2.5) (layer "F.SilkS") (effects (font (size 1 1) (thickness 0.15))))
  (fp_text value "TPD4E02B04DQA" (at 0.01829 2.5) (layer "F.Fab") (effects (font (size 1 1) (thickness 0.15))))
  (fp_line (start 0.5 -1.4) (end -0.8 -1.4) (layer "F.SilkS") (width 0.12))
  (fp_line (start 0.5 1.4) (end -0.5 1.4) (layer "F.SilkS") (width 0.12))
  (pad "1" smd rect (at -0.385 -1 270) (locked) (size 0.3 0.55) (layers "F.Cu" "F.Paste" "F.Mask") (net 27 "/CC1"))
  (pad "2" smd rect (at -0.385 -0.5 270) (locked) (size 0.3 0.55) (layers "F.Cu" "F.Paste" "F.Mask") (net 19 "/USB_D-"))
  (pad "3" smd rect (at -0.385 0 270) (locked) (size 0.4 0.55) (layers "F.Cu" "F.Paste" "F.Mask") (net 14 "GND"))
  (pad "4" smd rect (at -0.385 0.5 270) (locked) (size 0.3 0.55) (layers "F.Cu" "F.Paste" "F.Mask") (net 20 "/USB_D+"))
  (pad "5" smd rect (at -0.385 1 270) (locked) (size 0.3 0.55) (layers "F.Cu" "F.Paste" "F.Mask") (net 25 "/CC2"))
  (pad "6" smd rect (at 0.385 1 270) (locked) (size 0.3 0.55) (layers "F.Cu" "F.Paste" "F.Mask") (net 25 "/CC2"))
  (pad "7" smd rect (at 0.385 0.5 270) (locked) (size 0.3 0.55) (layers "F.Cu" "F.Paste" "F.Mask") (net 20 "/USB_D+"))
  (pad "8" smd rect (at 0.385 0 270) (locked) (size 0.4 0.55) (layers "F.Cu" "F.Paste" "F.Mask") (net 14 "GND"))
  (pad "9" smd rect (at 0.385 -0.5 270) (locked) (size 0.3 0.55) (layers "F.Cu" "F.Paste" "F.Mask") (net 19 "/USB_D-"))
  (pad "10" smd rect (at 0.385 -1 270) (locked) (size 0.3 0.55) (layers "F.Cu" "F.Paste" "F.Mask") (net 27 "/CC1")))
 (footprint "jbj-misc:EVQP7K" (layer "F.Cu") (at 75.5 55)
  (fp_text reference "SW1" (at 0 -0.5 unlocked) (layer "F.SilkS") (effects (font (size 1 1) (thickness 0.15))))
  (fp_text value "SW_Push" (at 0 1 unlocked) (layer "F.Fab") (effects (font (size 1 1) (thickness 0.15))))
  (pad "1" smd rect (at 1.8 -0.725) (locked) (size 1.4 1.05) (layers "F.Cu" "F.Paste" "F.Mask") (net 1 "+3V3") (clearance 0.01))
  (pad "1" smd rect (at -1.8 -0.725) (locked) (size 1.4 1.05) (layers "F.Cu" "F.Paste" "F.Mask") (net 1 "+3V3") (clearance 0.01))
  (pad "2" smd rect (at 1.8 0.725) (locked) (size 1.4 1.05) (layers "F.Cu" "F.Paste" "F.Mask") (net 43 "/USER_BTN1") (clearance 0.01))
  (pad "2" smd rect (at -1.8 0.725) (locked) (size 1.4 1.05) (layers "F.Cu" "F.Paste" "F.Mask") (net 43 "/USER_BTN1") (clearance 0.01)))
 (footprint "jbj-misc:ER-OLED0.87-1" (layer "B.Cu") (at 68.992 51.25 180)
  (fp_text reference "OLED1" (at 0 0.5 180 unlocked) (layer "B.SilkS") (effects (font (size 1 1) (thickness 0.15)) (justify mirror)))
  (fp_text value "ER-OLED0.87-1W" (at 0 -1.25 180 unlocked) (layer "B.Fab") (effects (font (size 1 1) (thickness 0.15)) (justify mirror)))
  (pad "1" smd rect (at 9.5 -4.03 90) (locked) (size 0.32 2) (layers "B.Cu" "B.Paste" "B.Mask") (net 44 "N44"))
  (pad "2" smd rect (at 9.5 -3.41 90) (locked) (size 0.32 2) (layers "B.Cu" "B.Paste" "B.Mask") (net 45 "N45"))
  (pad "3" smd rect (at 9.5 -2.79 90) (locked) (size 0.32 2) (layers "B.Cu" "B.Paste" "B.Mask") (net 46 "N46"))
  (pad "4" smd rect (at 9.5 -2.17 90) (locked) (size 0.32 2) (layers "B.Cu" "B.Paste" "B.Mask") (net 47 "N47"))
  (pad "5" smd rect (at 9.5 -1.55 90) (locked) (size 0.32 2) (layers "B.Cu" "B.Paste" "B.Mask") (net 1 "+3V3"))
  (pad "6" smd rect (at 9.5 -0.93 90) (locked) (size 0.32 2) (layers "B.Cu" "B.Paste" "B.Mask") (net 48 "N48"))
  (pad "7" smd rect (at 9.5 -0.31 90) (locked) (size 0.32 2) (layers "B.Cu" "B.Paste" "B.Mask") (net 14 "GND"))
  (pad "8" smd rect (at 9.5 0.31 90) (locked) (size 0.32 2) (layers "B.Cu" "B.Paste" "B.Mask") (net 1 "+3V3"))
  (pad "9" smd rect (at 9.5 0.93 90) (locked) (size 0.32 2) (layers "B.Cu" "B.Paste" "B.Mask") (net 23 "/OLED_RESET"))
  (pad "10" smd rect (at 9.5 1.55 90) (locked) (size 0.32 2) (layers "B.Cu" "B.Paste" "B.Mask") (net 16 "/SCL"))
  (pad "11" smd rect (at 9.5 2.17 90) (locked) (size 0.32 2) (layers "B.Cu" "B.Paste" "B.Mask") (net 26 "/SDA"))
  (pad "12" smd rect (at 9.5 2.79 90) (locked) (size 0.32 2) (layers "B.Cu" "B.Paste" "B.Mask") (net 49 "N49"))
  (pad "13" smd rect (at 9.5 3.41 90) (locked) (size 0.32 2) (layers "B.Cu" "B.Paste" "B.Mask") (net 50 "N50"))
  (pad "14" smd rect (at 9.5 4.03 90) (locked) (size 0.32 2) (layers "B.Cu" "B.Paste" "B.Mask") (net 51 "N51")))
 (gr_line (start 91.25 47.7) (end 91.25 45.5) (layer "Edge.Cuts") (width 0.1))
 (gr_line (start 91.25 45.5) (end 46 45.5) (layer "Edge.Cuts") (width 0.1))
 (gr_line (start 91.25 56.5) (end 91.25 54.3) (layer "Edge.Cuts") (width 0.1))
 (gr_line (start 46 45.5) (end 46 56.5) (layer "Edge.Cuts") (width 0.1))
 (gr_line (start 46 56.5) (end 91.25 56.5) (layer "Edge.Cuts") (width 0.1))
 (segment (start 54.615 50.5) (end 55.385 50.5) (width 0.2) (layer "F.Cu") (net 19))
 (segment (start 52.99 50.275) (end 53.3432 50.275) (width 0.2) (layer "F.Cu") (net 19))
 (segment (start 55.797501 50.5) (end 56.072501 50.775) (width 0.2) (layer "F.Cu") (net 19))
 (segment (start 52 50.25) (end 52.6 50.25) (width 0.127) (layer "F.Cu") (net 19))
 (segment (start 54.202499 50.5) (end 54.615 50.5) (width 0.2) (layer "F.Cu") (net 19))
 (segment (start 53.3432 50.275) (end 53.8432 50.775) (width 0.2) (layer "F.Cu") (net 19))
 (segment (start 55.385 50.5) (end 55.797501 50.5) (width 0.2) (layer "F.Cu") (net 19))
 (segment (start 51.75 50.5) (end 52 50.25) (width 0.127) (layer "F.Cu") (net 19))
 (segment (start 52 51.75) (end 51.75 51.5) (width 0.127) (layer "F.Cu") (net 19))
 (segment (start 51.75 51.5) (end 51.75 50.5) (width 0.127) (layer "F.Cu") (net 19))
 (segment (start 52.6 51.75) (end 52 51.75) (width 0.127) (layer "F.Cu") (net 19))
 (segment (start 56.072501 50.775) (end 57.5 50.775) (width 0.2) (layer "F.Cu") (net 19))
 (segment (start 52.965 50.25) (end 52.99 50.275) (width 0.2) (layer "F.Cu") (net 19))
 (segment (start 52.6 50.25) (end 52.965 50.25) (width 0.2) (layer "F.Cu") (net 19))
 (segment (start 53.8432 50.775) (end 53.927499 50.775) (width 0.2) (layer "F.Cu") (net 19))
 (segment (start 53.927499 50.775) (end 54.202499 50.5) (width 0.2) (layer "F.Cu") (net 19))
 (segment (start 55.385 51.5) (end 55.797501 51.5) (width 0.2) (layer "F.Cu") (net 20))
 (segment (start 53.6568 51.225) (end 53.927499 51.225) (width 0.2) (layer "F.Cu") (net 20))
 (segment (start 55.797501 51.5) (end 56.072501 51.225) (width 0.2) (layer "F.Cu") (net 20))
 (segment (start 52.6 51.25) (end 52.6 50.75) (width 0.0889) (layer "F.Cu") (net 20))
 (segment (start 52.965 50.75) (end 52.99 50.725) (width 0.2) (layer "F.Cu") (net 20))
 (segment (start 56.072501 51.225) (end 57.5 51.225) (width 0.2) (layer "F.Cu") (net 20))
 (segment (start 54.615 51.5) (end 55.385 51.5) (width 0.2) (layer "F.Cu") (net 20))
 (segment (start 52.6 50.75) (end 52.965 50.75) (width 0.2) (layer "F.Cu") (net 20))
 (segment (start 54.202499 51.5) (end 54.615 51.5) (width 0.2) (layer "F.Cu") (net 20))
 (segment (start 53.1568 50.725) (end 53.6568 51.225) (width 0.2) (layer "F.Cu") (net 20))
 (segment (start 53.927499 51.225) (end 54.202499 51.5) (width 0.2) (layer "F.Cu") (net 20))
 (segment (start 52.99 50.725) (end 53.1568 50.725) (width 0.2) (layer "F.Cu") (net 20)))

